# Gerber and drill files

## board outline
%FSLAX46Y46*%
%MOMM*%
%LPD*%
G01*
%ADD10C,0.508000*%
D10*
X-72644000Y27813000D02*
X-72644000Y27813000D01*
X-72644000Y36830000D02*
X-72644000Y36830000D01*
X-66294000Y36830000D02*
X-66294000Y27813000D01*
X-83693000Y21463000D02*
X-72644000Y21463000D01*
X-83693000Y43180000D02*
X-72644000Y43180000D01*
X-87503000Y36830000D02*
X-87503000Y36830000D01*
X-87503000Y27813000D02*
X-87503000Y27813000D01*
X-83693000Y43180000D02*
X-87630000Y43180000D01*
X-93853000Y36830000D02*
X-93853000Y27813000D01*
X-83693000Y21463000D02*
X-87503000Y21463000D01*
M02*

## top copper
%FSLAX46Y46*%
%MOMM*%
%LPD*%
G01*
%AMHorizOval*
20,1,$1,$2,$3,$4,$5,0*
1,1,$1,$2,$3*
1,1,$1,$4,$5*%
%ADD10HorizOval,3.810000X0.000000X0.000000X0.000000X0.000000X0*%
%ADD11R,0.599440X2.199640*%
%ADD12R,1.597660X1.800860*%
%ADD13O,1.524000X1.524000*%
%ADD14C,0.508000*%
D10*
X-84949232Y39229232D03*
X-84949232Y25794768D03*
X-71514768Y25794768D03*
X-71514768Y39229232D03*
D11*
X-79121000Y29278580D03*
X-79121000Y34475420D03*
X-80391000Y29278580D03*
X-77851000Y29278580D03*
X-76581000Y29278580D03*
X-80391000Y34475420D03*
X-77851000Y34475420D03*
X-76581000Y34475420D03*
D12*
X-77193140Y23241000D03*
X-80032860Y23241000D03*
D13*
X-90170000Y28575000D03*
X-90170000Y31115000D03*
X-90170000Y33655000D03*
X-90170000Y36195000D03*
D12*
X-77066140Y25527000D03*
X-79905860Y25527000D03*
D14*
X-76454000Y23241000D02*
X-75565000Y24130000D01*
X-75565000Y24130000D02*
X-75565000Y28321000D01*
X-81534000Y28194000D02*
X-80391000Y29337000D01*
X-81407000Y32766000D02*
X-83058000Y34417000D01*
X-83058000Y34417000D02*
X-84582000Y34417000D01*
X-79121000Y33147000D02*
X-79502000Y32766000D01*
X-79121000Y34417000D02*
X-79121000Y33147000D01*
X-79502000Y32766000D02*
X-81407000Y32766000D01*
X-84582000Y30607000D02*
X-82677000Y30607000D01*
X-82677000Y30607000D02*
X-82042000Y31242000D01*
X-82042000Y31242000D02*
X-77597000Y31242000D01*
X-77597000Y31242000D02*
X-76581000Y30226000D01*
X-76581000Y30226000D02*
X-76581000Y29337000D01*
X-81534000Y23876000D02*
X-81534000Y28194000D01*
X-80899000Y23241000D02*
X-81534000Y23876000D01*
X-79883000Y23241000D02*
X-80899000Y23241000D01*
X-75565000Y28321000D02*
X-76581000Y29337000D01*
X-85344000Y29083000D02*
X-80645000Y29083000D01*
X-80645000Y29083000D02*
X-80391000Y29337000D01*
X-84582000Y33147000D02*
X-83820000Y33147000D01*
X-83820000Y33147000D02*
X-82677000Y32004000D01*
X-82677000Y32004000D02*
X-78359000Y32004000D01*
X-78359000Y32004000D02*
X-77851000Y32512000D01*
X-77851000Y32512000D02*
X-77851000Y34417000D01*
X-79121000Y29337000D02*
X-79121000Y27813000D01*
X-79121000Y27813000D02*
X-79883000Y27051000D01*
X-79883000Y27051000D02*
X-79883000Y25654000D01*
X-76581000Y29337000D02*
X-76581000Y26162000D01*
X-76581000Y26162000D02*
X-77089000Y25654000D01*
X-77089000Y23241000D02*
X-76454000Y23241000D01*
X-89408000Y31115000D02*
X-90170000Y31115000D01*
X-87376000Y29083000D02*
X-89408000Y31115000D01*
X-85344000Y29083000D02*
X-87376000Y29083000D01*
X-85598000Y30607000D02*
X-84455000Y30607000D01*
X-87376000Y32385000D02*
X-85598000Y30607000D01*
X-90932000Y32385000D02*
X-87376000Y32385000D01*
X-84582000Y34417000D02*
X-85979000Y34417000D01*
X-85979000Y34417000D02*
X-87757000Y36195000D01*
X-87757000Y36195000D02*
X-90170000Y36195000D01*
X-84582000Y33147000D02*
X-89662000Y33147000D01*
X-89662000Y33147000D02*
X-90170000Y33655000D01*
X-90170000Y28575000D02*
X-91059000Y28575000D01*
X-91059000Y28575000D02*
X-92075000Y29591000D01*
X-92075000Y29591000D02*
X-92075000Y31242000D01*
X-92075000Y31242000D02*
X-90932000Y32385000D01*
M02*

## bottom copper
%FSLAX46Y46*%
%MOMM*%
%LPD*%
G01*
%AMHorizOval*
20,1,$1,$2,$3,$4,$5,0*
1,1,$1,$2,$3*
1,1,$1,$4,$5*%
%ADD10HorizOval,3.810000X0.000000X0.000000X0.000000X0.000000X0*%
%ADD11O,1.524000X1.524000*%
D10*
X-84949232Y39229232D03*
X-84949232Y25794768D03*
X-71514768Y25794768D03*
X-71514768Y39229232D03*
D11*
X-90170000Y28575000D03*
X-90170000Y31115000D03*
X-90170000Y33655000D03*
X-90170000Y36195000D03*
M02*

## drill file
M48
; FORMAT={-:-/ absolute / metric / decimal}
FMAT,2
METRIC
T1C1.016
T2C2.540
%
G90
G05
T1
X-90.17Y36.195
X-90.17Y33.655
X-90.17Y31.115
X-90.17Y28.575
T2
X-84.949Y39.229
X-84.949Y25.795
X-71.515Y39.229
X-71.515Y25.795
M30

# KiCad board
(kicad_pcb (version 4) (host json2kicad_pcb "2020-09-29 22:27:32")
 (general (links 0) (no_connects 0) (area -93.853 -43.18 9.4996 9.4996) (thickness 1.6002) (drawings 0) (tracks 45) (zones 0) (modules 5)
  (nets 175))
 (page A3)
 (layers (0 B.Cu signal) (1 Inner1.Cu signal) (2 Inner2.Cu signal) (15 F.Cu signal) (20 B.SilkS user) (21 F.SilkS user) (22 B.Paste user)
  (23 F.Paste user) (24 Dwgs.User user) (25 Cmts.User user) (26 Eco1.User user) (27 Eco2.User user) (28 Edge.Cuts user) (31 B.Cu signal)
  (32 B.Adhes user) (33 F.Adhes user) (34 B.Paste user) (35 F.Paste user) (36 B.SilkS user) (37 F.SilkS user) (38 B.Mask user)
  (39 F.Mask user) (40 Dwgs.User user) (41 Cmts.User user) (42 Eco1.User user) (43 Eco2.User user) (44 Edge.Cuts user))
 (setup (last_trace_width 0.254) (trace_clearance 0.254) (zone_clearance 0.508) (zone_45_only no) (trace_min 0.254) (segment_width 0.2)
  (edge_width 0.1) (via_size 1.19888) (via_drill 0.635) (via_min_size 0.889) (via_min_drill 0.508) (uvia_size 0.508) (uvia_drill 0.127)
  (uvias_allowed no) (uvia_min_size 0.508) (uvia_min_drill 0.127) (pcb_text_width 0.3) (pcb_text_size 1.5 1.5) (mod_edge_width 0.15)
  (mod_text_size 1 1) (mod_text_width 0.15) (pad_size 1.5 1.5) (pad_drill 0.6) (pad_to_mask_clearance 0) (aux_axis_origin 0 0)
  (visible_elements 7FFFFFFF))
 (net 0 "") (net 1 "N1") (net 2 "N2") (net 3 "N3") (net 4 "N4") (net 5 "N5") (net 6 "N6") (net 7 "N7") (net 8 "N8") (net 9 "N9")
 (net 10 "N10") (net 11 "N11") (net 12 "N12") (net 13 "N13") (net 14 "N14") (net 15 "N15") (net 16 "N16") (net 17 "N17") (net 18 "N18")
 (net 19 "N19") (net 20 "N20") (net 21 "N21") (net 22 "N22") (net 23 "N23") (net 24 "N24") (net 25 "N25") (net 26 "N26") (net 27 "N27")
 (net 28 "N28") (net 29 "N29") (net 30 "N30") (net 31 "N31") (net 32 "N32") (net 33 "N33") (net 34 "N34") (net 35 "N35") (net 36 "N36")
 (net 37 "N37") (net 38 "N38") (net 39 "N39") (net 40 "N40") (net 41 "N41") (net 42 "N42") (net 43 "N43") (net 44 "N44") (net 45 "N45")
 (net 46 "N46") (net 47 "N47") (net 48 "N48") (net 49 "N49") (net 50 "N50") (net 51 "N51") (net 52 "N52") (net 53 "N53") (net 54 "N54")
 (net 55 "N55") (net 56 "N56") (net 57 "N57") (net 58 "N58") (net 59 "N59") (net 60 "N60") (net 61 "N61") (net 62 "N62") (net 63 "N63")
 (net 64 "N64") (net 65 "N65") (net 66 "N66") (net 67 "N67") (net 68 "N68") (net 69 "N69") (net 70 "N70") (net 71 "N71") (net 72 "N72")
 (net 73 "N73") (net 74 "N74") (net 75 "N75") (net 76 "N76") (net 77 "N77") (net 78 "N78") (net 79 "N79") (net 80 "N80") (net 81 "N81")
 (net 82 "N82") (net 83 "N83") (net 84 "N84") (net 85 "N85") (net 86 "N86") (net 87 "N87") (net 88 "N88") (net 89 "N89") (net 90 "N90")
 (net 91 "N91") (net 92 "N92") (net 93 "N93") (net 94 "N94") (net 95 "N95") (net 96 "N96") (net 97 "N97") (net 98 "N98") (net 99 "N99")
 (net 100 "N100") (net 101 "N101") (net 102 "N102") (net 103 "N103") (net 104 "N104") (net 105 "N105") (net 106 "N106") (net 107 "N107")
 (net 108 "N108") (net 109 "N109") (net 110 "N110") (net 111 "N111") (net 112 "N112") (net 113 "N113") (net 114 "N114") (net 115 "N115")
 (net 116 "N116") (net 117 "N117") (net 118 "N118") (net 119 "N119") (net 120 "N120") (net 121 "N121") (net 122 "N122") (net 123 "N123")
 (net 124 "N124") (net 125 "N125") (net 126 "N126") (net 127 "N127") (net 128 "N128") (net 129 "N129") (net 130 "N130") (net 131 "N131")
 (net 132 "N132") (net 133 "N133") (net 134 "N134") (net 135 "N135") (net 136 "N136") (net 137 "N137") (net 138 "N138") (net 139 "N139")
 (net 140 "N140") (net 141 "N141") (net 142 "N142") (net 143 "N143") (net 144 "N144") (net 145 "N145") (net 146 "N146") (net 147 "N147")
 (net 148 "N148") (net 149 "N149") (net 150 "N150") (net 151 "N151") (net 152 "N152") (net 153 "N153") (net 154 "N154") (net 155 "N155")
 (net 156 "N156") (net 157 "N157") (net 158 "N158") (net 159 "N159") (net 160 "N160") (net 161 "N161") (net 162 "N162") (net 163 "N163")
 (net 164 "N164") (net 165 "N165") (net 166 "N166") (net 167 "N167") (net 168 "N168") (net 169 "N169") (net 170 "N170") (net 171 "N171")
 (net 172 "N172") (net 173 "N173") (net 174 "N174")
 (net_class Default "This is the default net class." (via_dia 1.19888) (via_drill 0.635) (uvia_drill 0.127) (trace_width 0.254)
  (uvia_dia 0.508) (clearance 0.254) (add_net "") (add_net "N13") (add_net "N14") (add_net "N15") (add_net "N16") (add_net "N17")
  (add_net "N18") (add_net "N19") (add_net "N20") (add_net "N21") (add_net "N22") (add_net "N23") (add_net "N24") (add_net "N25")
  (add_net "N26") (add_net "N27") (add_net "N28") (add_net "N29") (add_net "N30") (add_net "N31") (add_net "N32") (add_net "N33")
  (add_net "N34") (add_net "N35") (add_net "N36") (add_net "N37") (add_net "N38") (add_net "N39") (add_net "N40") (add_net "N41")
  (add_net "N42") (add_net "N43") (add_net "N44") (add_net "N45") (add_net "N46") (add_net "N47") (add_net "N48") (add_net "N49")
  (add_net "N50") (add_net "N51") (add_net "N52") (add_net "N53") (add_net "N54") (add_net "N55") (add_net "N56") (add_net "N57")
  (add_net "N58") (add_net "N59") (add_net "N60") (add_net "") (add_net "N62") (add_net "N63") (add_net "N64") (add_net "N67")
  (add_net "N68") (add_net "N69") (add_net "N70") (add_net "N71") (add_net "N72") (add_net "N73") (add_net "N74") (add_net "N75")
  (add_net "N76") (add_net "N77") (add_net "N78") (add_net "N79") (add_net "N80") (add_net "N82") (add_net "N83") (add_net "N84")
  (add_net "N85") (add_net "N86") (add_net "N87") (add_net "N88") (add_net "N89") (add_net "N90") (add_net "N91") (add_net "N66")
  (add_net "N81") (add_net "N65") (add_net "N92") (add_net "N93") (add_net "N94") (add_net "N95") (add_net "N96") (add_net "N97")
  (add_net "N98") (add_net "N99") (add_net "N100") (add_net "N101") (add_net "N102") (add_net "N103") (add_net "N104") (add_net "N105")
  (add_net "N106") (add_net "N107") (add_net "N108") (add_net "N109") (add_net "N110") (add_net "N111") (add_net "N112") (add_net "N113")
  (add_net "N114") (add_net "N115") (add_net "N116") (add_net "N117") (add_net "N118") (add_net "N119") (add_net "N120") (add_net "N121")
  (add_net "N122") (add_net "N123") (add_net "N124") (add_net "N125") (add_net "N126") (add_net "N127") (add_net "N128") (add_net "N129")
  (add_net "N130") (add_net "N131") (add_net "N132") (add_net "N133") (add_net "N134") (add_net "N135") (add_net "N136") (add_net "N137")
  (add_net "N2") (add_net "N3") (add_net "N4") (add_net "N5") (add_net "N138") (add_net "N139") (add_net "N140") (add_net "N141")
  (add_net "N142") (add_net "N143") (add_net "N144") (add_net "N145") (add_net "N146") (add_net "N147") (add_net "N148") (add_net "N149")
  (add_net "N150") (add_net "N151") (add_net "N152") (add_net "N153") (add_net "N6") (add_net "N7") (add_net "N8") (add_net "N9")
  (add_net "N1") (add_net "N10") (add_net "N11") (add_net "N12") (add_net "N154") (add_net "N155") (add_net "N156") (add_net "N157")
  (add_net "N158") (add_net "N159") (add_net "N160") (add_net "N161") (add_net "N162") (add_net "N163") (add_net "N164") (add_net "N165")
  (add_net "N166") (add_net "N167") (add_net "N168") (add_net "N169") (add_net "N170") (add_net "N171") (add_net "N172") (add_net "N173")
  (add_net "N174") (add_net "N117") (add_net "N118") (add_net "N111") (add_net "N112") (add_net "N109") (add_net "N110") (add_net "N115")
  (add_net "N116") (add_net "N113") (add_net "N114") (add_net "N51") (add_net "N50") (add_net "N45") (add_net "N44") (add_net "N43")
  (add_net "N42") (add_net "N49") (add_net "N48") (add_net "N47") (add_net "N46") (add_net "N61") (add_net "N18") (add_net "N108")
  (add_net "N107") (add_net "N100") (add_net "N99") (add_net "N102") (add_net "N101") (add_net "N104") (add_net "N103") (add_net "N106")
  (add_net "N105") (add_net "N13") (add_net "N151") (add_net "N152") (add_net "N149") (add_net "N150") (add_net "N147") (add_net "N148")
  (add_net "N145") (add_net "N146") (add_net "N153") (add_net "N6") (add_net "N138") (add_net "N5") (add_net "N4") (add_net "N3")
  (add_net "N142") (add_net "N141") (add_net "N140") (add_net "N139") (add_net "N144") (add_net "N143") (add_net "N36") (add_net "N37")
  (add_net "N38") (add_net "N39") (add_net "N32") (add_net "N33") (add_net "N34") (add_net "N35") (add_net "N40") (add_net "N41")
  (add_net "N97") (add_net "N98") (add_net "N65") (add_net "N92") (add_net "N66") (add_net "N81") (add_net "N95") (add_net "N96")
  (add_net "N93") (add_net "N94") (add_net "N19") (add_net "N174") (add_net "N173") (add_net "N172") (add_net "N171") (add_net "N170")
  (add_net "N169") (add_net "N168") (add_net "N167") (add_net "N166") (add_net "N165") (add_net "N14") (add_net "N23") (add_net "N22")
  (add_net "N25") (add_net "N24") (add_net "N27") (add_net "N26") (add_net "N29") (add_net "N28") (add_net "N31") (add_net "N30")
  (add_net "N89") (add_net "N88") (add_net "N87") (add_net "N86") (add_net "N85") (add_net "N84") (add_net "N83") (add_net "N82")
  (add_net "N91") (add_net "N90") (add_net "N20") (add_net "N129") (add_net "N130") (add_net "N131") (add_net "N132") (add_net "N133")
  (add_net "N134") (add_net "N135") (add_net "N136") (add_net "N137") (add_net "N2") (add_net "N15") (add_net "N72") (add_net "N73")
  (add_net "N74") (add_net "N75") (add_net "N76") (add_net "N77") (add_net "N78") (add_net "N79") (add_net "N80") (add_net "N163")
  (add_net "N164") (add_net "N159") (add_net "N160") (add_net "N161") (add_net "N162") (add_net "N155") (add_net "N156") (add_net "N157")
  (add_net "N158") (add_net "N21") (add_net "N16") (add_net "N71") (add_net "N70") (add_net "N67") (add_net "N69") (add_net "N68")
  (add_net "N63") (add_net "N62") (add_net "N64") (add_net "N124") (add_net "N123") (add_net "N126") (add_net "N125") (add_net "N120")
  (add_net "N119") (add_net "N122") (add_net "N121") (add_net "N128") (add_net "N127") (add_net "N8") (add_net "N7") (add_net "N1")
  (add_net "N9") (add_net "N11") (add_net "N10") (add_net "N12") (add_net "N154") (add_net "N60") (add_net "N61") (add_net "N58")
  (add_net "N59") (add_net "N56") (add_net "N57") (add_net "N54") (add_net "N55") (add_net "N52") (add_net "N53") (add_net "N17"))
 (segment (start -76.454 -23.241) (end -75.565 -24.13) (width 0.508) (layer F.Cu) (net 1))
 (gr_line (start -72.644 -27.813) (end -72.644 -27.813) (angle -90.00) (width 0.508) (layer Edge.Cuts))
 (gr_line (start -72.644 -36.83) (end -72.644 -36.83) (angle -90.00) (width 0.508) (layer Edge.Cuts))
 (segment (start -75.565 -24.13) (end -75.565 -28.321) (width 0.508) (layer F.Cu) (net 1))
 (gr_line (start -66.294 -36.83) (end -66.294 -27.813) (angle 51566.20) (width 0.508) (layer Edge.Cuts))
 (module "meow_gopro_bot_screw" (layer "F.Cu") (at -78.232 -32.512 -135.00)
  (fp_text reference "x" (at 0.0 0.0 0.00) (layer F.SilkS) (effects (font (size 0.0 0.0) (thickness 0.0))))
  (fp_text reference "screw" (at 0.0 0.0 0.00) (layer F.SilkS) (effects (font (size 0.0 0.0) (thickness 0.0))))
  (pad S0 thru_hole oval (at 0.0 9.4996 -135.00) (size 3.81 3.81) (drill 2.54)
   (layers "B.Cu" "Inner1.Cu" "Inner2.Cu" "F.Cu" "B.Paste" "F.Paste") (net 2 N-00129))
  (pad S1 thru_hole oval (at 9.4996 0.0 -135.00) (size 3.81 3.81) (drill 2.54)
   (layers "B.Cu" "Inner1.Cu" "Inner2.Cu" "F.Cu" "B.Paste" "F.Paste") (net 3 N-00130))
  (pad S2 thru_hole oval (at 0.0 -9.4996 -135.00) (size 3.81 3.81) (drill 2.54)
   (layers "B.Cu" "Inner1.Cu" "Inner2.Cu" "F.Cu" "B.Paste" "F.Paste") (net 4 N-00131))
  (pad S3 thru_hole oval (at -9.4996 0.0 -135.00) (size 3.81 3.81) (drill 2.54)
   (layers "B.Cu" "Inner1.Cu" "Inner2.Cu" "F.Cu" "B.Paste" "F.Paste") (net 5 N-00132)))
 (gr_line (start -83.693 -21.463) (end -72.644 -21.463) (angle 51566.20) (width 0.508) (layer Edge.Cuts))
 (gr_line (start -83.693 -43.18) (end -72.644 -43.18) (angle 51566.20) (width 0.508) (layer Edge.Cuts))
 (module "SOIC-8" (layer "F.Cu") (at -78.486 -31.877 0.00)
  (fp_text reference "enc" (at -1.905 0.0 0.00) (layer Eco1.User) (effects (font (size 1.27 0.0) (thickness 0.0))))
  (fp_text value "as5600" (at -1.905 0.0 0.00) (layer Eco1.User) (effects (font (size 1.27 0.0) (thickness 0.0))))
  (pad 2 smd rect (at -0.635 2.59842 0.00) (size 0.59944 2.19964) (drill 0.0) (layers "F.Cu" "F.Paste") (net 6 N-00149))
  (pad 7 smd rect (at -0.635 -2.59842 0.00) (size 0.59944 2.19964) (drill 0.0) (layers "F.Cu" "F.Paste") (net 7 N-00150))
  (pad 1 smd rect (at -1.905 2.59842 0.00) (size 0.59944 2.19964) (drill 0.0) (layers "F.Cu" "F.Paste") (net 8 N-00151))
  (pad 3 smd rect (at 0.635 2.59842 0.00) (size 0.59944 2.19964) (drill 0.0) (layers "F.Cu" "F.Paste") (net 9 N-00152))
  (pad 4 smd rect (at 1.905 2.59842 0.00) (size 0.59944 2.19964) (drill 0.0) (layers "F.Cu" "F.Paste") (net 1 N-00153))
  (pad 8 smd rect (at -1.905 -2.59842 0.00) (size 0.59944 2.19964) (drill 0.0) (layers "F.Cu" "F.Paste") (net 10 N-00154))
  (pad 6 smd rect (at 0.635 -2.59842 0.00) (size 0.59944 2.19964) (drill 0.0) (layers "F.Cu" "F.Paste") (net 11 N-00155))
  (pad 5 smd rect (at 1.905 -2.59842 0.00) (size 0.59944 2.19964) (drill 0.0) (layers "F.Cu" "F.Paste") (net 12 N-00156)))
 (segment (start -81.534 -28.194) (end -80.391 -29.337) (width 0.508) (layer F.Cu) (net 8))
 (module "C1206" (layer "F.Cu") (at -78.613 -23.241 0.00)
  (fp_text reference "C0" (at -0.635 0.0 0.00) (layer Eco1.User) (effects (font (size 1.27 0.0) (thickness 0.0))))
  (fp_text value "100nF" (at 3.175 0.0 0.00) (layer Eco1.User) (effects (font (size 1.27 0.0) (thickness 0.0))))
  (pad 2 smd rect (at 1.41986 0.0 0.00) (size 1.59766 1.80086) (drill 0.0) (layers "F.Cu" "F.Paste") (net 1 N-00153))
  (pad 1 smd rect (at -1.41986 0.0 0.00) (size 1.59766 1.80086) (drill 0.0) (layers "F.Cu" "F.Paste") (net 8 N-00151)))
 (segment (start -81.407 -32.766) (end -83.058 -34.417) (width 0.508) (layer F.Cu) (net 7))
 (segment (start -83.058 -34.417) (end -84.582 -34.417) (width 0.508) (layer F.Cu) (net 7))
 (segment (start -79.121 -33.147) (end -79.502 -32.766) (width 0.508) (layer F.Cu) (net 7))
 (segment (start -79.121 -34.417) (end -79.121 -33.147) (width 0.508) (layer F.Cu) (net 7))
 (segment (start -79.502 -32.766) (end -81.407 -32.766) (width 0.508) (layer F.Cu) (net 7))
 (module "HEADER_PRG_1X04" (layer "F.Cu") (at -90.17 -32.385 90.00)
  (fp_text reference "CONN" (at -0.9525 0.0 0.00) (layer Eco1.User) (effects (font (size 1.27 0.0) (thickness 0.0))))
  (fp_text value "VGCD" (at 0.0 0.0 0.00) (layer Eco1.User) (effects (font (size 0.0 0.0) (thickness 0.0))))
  (pad 1 thru_hole oval (at -3.81 0.0 90.00) (size 1.524 1.524) (drill 1.016)
   (layers "B.Cu" "Inner1.Cu" "Inner2.Cu" "F.Cu" "B.Paste" "F.Paste") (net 1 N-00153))
  (pad 2 thru_hole oval (at -1.27 0.0 90.00) (size 1.524 1.524) (drill 1.016)
   (layers "B.Cu" "Inner1.Cu" "Inner2.Cu" "F.Cu" "B.Paste" "F.Paste") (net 8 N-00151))
  (pad 3 thru_hole oval (at 1.27 0.0 90.00) (size 1.524 1.524) (drill 1.016)
   (layers "B.Cu" "Inner1.Cu" "Inner2.Cu" "F.Cu" "B.Paste" "F.Paste") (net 11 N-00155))
  (pad 4 thru_hole oval (at 3.81 0.0 90.00) (size 1.524 1.524) (drill 1.016)
   (layers "B.Cu" "Inner1.Cu" "Inner2.Cu" "F.Cu" "B.Paste" "F.Paste") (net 7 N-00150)))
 (segment (start -84.582 -30.607) (end -82.677 -30.607) (width 0.508) (layer F.Cu) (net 1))
 (segment (start -82.677 -30.607) (end -82.042 -31.242) (width 0.508) (layer F.Cu) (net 1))
 (segment (start -82.042 -31.242) (end -77.597 -31.242) (width 0.508) (layer F.Cu) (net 1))
 (segment (start -77.597 -31.242) (end -76.581 -30.226) (width 0.508) (layer F.Cu) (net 1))
 (segment (start -76.581 -30.226) (end -76.581 -29.337) (width 0.508) (layer F.Cu) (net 1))
 (segment (start -81.534 -23.876) (end -81.534 -28.194) (width 0.508) (layer F.Cu) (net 8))
 (segment (start -80.899 -23.241) (end -81.534 -23.876) (width 0.508) (layer F.Cu) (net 8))
 (segment (start -79.883 -23.241) (end -80.899 -23.241) (width 0.508) (layer F.Cu) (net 8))
 (segment (start -75.565 -28.321) (end -76.581 -29.337) (width 0.508) (layer F.Cu) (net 1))
 (segment (start -85.344 -29.083) (end -80.645 -29.083) (width 0.508) (layer F.Cu) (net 8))
 (segment (start -80.645 -29.083) (end -80.391 -29.337) (width 0.508) (layer F.Cu) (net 8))
 (segment (start -84.582 -33.147) (end -83.82 -33.147) (width 0.508) (layer F.Cu) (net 11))
 (segment (start -83.82 -33.147) (end -82.677 -32.004) (width 0.508) (layer F.Cu) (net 11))
 (segment (start -82.677 -32.004) (end -78.359 -32.004) (width 0.508) (layer F.Cu) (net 11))
 (segment (start -78.359 -32.004) (end -77.851 -32.512) (width 0.508) (layer F.Cu) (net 11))
 (segment (start -77.851 -32.512) (end -77.851 -34.417) (width 0.508) (layer F.Cu) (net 11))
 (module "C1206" (layer "F.Cu") (at -78.486 -25.527 0.00)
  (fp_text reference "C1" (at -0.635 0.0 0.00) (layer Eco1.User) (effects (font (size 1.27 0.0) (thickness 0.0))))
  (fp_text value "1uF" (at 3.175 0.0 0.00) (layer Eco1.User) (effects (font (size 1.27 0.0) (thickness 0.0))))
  (pad 2 smd rect (at 1.41986 0.0 0.00) (size 1.59766 1.80086) (drill 0.0) (layers "F.Cu" "F.Paste") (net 1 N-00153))
  (pad 1 smd rect (at -1.41986 0.0 0.00) (size 1.59766 1.80086) (drill 0.0) (layers "F.Cu" "F.Paste") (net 6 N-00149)))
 (segment (start -79.121 -29.337) (end -79.121 -27.813) (width 0.508) (layer F.Cu) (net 6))
 (segment (start -79.121 -27.813) (end -79.883 -27.051) (width 0.508) (layer F.Cu) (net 6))
 (segment (start -79.883 -27.051) (end -79.883 -25.654) (width 0.508) (layer F.Cu) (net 6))
 (segment (start -76.581 -29.337) (end -76.581 -26.162) (width 0.508) (layer F.Cu) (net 1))
 (segment (start -76.581 -26.162) (end -77.089 -25.654) (width 0.508) (layer F.Cu) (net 1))
 (segment (start -77.089 -23.241) (end -76.454 -23.241) (width 0.508) (layer F.Cu) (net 1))
 (segment (start -89.408 -31.115) (end -90.17 -31.115) (width 0.508) (layer F.Cu) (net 8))
 (segment (start -87.376 -29.083) (end -89.408 -31.115) (width 0.508) (layer F.Cu) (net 8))
 (segment (start -85.344 -29.083) (end -87.376 -29.083) (width 0.508) (layer F.Cu) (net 8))
 (segment (start -85.598 -30.607) (end -84.455 -30.607) (width 0.508) (layer F.Cu) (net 1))
 (gr_line (start -87.503 -36.83) (end -87.503 -36.83) (angle -90.00) (width 0.508) (layer Edge.Cuts))
 (segment (start -87.376 -32.385) (end -85.598 -30.607) (width 0.508) (layer F.Cu) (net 1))
 (segment (start -90.932 -32.385) (end -87.376 -32.385) (width 0.508) (layer F.Cu) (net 1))
 (gr_line (start -87.503 -27.813) (end -87.503 -27.813) (angle -90.00) (width 0.508) (layer Edge.Cuts))
 (gr_line (start -83.693 -43.18) (end -87.63 -43.18) (angle 51566.20) (width 0.508) (layer Edge.Cuts))
 (gr_line (start -93.853 -36.83) (end -93.853 -27.813) (angle 51566.20) (width 0.508) (layer Edge.Cuts))
 (gr_line (start -83.693 -21.463) (end -87.503 -21.463) (angle 51566.20) (width 0.508) (layer Edge.Cuts))
 (segment (start -84.582 -34.417) (end -85.979 -34.417) (width 0.508) (layer F.Cu) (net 7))
 (segment (start -85.979 -34.417) (end -87.757 -36.195) (width 0.508) (layer F.Cu) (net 7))
 (segment (start -87.757 -36.195) (end -90.17 -36.195) (width 0.508) (layer F.Cu) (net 7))
 (segment (start -84.582 -33.147) (end -89.662 -33.147) (width 0.508) (layer F.Cu) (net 11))
 (segment (start -89.662 -33.147) (end -90.17 -33.655) (width 0.508) (layer F.Cu) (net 11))
 (segment (start -90.17 -28.575) (end -91.059 -28.575) (width 0.508) (layer F.Cu) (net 1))
 (segment (start -91.059 -28.575) (end -92.075 -29.591) (width 0.508) (layer F.Cu) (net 1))
 (segment (start -92.075 -29.591) (end -92.075 -31.242) (width 0.508) (layer F.Cu) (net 1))
 (segment (start -92.075 -31.242) (end -90.932 -32.385) (width 0.508) (layer F.Cu) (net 1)))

